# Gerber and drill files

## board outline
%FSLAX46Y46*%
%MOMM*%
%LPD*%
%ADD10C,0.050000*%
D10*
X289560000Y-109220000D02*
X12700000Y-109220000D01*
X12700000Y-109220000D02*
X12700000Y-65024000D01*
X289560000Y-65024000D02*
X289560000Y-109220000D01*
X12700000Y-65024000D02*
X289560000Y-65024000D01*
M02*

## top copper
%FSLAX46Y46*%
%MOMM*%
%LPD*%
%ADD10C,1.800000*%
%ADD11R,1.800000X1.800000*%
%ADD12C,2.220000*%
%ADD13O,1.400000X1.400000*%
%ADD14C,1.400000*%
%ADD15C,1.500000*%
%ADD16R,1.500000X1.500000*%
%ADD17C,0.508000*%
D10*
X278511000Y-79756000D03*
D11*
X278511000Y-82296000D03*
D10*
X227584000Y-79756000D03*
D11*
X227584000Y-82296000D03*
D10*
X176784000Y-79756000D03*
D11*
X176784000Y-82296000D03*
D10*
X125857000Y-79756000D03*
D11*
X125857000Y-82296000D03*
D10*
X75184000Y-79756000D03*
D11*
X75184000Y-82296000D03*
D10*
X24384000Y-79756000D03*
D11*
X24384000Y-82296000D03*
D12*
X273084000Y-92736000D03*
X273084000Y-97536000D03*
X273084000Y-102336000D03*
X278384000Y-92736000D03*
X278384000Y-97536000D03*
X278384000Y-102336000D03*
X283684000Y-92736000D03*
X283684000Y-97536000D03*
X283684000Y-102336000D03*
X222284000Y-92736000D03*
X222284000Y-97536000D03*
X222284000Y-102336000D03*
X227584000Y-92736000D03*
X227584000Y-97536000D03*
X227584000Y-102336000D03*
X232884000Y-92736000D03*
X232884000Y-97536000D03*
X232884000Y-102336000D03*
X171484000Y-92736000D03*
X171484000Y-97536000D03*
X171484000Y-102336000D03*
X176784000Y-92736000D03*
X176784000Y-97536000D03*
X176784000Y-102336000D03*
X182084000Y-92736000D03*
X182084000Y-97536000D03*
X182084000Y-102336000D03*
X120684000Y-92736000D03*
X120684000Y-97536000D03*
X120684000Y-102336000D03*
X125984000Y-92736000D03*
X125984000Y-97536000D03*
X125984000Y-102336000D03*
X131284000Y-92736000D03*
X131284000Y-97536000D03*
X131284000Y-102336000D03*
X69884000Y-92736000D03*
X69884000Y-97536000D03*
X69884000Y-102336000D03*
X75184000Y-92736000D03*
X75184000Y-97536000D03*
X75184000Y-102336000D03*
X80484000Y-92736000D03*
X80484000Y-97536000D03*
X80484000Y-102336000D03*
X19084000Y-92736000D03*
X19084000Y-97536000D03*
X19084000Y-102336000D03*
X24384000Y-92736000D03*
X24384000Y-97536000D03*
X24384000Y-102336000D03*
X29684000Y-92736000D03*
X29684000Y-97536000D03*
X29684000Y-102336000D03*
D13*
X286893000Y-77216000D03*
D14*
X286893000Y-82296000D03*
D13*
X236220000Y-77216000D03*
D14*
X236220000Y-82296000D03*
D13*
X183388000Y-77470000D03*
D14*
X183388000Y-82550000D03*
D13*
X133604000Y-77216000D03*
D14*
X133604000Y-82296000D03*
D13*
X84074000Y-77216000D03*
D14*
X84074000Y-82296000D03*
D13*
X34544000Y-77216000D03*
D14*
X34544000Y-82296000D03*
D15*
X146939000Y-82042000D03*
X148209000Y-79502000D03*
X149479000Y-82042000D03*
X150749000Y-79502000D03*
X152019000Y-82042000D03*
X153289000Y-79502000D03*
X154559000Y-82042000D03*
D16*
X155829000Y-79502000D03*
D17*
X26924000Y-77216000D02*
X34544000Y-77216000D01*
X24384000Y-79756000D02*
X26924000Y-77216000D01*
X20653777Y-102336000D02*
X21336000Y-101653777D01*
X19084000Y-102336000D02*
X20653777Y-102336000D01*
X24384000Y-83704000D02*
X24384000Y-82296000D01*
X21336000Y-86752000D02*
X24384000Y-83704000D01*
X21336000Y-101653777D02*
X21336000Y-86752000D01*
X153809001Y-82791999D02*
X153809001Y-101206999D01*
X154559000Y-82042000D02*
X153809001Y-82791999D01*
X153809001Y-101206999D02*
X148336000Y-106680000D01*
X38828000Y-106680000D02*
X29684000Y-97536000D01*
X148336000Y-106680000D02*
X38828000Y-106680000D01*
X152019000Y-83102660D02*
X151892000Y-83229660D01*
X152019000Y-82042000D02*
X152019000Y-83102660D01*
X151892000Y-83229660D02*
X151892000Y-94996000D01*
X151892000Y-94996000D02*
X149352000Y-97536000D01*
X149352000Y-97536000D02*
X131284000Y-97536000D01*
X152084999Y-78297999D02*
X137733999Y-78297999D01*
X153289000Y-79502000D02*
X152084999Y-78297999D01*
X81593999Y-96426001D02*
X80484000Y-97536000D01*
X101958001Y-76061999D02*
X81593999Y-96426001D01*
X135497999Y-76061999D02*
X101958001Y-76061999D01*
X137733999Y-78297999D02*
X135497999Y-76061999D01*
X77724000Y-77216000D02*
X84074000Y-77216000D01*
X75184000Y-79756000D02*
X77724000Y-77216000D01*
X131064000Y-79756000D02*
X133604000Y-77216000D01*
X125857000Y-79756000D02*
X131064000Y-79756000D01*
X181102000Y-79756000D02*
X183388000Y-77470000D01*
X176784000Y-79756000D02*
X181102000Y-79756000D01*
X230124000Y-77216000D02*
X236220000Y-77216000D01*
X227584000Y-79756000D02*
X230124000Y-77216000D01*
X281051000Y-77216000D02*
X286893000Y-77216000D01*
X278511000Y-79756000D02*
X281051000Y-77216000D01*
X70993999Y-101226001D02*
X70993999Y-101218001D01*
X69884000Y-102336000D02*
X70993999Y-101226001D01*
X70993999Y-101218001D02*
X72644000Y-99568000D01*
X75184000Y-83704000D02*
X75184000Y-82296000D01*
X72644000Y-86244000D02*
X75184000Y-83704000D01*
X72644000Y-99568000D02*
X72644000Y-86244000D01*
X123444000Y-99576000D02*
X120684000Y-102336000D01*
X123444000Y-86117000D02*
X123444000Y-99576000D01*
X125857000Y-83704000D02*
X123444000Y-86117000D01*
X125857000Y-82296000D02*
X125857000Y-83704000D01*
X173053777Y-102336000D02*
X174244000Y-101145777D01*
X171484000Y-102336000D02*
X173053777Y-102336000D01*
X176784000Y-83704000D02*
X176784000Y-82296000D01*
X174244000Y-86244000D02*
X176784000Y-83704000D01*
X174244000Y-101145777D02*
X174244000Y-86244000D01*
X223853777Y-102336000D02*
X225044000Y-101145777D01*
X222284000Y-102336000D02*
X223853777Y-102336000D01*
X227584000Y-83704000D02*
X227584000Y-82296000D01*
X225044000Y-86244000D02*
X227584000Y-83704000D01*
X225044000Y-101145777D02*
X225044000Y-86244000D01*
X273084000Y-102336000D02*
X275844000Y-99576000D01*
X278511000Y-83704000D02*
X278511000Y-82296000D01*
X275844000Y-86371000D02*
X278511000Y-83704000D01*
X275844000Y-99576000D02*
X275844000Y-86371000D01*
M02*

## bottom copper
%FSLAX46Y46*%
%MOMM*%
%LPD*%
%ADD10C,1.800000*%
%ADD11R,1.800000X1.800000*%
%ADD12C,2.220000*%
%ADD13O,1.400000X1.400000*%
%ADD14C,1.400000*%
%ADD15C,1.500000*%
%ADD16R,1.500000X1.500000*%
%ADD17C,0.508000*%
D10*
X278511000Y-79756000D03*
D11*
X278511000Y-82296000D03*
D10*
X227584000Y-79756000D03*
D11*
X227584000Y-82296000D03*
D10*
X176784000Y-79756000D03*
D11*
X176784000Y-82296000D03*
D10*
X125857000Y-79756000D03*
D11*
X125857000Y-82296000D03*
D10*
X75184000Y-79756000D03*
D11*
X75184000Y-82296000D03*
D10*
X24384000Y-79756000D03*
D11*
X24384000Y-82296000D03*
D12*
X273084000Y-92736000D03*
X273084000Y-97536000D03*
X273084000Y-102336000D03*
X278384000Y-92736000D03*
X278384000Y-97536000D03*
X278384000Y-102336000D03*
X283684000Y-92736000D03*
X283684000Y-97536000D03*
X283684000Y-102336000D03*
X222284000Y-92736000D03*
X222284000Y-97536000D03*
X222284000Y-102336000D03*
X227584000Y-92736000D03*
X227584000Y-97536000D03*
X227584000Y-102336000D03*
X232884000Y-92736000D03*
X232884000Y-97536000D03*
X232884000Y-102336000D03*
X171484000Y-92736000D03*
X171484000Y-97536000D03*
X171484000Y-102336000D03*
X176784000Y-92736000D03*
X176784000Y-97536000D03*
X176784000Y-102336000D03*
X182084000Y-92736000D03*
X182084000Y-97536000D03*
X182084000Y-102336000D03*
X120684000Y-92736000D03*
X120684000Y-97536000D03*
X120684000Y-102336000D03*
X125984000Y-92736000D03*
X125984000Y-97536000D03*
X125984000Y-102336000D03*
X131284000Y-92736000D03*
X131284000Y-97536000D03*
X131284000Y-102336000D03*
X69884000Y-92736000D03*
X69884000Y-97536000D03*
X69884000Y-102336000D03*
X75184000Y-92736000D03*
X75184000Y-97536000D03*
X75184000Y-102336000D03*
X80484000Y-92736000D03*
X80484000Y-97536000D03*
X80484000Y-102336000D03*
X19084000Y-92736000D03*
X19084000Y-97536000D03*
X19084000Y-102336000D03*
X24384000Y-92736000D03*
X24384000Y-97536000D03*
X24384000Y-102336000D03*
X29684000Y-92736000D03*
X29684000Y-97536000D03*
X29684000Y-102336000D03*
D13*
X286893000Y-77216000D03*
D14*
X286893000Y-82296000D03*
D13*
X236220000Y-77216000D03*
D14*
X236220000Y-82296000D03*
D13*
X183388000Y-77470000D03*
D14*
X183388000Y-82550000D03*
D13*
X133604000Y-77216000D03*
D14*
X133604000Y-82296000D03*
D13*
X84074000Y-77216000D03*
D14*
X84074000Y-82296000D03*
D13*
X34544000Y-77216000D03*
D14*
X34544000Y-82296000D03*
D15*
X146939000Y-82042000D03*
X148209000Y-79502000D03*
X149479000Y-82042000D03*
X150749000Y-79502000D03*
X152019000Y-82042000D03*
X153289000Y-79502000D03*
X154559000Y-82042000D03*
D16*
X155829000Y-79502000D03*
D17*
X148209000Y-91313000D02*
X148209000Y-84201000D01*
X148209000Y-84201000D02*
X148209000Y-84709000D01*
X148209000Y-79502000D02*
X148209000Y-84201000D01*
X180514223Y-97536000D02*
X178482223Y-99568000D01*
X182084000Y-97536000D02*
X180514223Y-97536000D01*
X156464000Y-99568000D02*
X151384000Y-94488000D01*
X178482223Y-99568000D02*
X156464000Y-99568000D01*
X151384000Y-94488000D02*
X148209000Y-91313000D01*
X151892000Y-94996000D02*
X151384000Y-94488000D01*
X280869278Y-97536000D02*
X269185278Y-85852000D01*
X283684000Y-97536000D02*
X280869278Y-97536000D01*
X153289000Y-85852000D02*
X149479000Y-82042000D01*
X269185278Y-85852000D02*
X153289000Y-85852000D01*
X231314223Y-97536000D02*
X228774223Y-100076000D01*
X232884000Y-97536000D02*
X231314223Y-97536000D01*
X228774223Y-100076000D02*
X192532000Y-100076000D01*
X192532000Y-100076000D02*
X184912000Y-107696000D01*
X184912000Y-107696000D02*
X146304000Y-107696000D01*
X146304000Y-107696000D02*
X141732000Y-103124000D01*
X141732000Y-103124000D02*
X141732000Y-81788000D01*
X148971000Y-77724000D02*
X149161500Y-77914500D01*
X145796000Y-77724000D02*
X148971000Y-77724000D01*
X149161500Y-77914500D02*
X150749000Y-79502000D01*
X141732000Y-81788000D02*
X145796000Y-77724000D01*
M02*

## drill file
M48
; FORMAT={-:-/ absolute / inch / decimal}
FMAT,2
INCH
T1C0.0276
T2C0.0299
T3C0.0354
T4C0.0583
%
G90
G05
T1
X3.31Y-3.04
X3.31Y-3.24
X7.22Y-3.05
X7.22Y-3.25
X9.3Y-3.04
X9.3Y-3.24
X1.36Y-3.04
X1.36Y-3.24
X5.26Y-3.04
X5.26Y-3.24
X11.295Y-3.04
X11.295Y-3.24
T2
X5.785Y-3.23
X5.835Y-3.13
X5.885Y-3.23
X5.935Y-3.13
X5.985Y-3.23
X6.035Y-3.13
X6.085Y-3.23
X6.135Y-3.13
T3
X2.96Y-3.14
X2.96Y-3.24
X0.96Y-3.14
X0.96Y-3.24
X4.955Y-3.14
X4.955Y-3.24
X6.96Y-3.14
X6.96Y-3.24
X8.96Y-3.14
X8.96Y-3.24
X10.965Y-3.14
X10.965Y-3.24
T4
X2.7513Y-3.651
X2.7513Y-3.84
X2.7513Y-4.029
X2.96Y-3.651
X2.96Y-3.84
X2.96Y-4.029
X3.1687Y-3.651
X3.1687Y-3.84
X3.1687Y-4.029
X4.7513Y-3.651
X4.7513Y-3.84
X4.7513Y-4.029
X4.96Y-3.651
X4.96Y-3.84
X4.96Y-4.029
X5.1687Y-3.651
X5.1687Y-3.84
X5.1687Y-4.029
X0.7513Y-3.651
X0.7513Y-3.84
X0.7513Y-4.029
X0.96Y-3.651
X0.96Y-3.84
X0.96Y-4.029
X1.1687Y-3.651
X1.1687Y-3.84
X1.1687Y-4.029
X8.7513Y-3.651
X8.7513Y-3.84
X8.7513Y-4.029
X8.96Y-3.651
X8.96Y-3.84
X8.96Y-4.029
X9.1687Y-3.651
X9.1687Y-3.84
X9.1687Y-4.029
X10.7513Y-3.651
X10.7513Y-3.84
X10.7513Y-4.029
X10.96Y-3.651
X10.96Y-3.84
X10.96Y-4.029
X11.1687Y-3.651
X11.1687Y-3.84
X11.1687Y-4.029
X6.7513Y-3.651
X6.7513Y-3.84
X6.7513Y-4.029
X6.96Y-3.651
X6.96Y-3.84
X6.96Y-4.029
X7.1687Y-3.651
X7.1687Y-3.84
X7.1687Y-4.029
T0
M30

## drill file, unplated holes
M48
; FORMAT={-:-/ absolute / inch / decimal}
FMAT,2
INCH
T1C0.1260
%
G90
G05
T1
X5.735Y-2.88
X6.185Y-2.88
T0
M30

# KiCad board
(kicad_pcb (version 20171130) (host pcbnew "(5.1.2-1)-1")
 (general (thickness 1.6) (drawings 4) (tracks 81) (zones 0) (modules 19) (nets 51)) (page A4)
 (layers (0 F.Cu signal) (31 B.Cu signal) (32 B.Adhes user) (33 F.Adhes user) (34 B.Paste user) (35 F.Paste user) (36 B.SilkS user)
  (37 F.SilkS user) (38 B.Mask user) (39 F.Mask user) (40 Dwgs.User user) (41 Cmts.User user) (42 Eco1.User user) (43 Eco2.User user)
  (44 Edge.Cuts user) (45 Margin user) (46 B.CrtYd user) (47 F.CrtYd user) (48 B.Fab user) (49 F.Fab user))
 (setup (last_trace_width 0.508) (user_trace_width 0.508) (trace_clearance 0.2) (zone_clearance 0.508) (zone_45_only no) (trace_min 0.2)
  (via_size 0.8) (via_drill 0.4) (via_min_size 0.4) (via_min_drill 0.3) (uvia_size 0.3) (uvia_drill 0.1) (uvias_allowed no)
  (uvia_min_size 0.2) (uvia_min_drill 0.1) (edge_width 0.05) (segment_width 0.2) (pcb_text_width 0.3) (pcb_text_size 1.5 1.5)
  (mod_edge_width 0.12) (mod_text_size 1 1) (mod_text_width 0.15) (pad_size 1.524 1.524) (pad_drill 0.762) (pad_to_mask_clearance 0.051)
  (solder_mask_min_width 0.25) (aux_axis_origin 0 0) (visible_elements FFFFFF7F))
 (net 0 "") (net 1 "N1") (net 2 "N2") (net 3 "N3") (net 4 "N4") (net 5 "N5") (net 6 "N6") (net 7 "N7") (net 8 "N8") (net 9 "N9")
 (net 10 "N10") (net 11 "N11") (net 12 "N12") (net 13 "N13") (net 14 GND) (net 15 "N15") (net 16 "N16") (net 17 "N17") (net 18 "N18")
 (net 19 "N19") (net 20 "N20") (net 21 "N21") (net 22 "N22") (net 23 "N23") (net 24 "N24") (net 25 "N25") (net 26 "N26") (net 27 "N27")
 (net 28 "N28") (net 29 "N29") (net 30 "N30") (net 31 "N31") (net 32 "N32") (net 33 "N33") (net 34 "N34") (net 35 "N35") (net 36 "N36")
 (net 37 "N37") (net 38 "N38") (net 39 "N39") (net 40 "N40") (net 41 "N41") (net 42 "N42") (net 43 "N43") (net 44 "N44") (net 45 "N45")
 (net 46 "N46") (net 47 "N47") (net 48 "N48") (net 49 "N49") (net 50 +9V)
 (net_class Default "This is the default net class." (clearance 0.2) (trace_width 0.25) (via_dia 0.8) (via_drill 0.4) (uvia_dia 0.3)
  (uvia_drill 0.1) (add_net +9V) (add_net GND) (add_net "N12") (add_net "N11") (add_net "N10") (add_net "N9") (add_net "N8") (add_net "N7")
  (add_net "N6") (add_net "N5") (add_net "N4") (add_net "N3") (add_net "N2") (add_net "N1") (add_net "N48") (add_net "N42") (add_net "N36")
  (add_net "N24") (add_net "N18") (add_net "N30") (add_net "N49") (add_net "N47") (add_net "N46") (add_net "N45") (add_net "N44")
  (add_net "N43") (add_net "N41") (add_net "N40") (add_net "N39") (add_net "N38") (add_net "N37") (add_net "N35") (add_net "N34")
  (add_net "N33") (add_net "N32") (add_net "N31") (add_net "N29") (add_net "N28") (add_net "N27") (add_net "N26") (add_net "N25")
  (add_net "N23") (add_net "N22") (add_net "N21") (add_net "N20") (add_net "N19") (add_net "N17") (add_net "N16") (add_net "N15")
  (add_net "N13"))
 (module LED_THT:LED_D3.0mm (layer F.Cu) (at 278.511 82.296 90)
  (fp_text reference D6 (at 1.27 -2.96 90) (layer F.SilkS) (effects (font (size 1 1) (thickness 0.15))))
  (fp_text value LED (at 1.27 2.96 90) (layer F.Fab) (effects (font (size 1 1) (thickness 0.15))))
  (pad 2 thru_hole circle (at 2.54 0 90) (size 1.8 1.8) (drill 0.9) (layers *.Cu *.Mask) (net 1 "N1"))
  (pad 1 thru_hole rect (at 0 0 90) (size 1.8 1.8) (drill 0.9) (layers *.Cu *.Mask) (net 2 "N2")))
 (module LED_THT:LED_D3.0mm (layer F.Cu) (at 227.584 82.296 90)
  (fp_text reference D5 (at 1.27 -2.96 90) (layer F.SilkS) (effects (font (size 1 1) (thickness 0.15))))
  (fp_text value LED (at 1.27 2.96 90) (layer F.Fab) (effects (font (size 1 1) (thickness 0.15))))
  (pad 2 thru_hole circle (at 2.54 0 90) (size 1.8 1.8) (drill 0.9) (layers *.Cu *.Mask) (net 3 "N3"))
  (pad 1 thru_hole rect (at 0 0 90) (size 1.8 1.8) (drill 0.9) (layers *.Cu *.Mask) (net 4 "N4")))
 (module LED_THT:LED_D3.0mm (layer F.Cu) (at 176.784 82.296 90)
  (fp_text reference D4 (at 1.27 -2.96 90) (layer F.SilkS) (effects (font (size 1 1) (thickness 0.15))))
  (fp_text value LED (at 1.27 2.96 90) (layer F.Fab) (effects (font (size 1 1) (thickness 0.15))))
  (pad 2 thru_hole circle (at 2.54 0 90) (size 1.8 1.8) (drill 0.9) (layers *.Cu *.Mask) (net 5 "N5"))
  (pad 1 thru_hole rect (at 0 0 90) (size 1.8 1.8) (drill 0.9) (layers *.Cu *.Mask) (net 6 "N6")))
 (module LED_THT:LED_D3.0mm (layer F.Cu) (at 125.857 82.296 90)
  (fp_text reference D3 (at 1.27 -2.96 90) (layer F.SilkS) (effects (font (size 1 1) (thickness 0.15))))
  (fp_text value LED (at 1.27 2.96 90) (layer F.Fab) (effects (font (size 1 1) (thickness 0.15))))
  (pad 2 thru_hole circle (at 2.54 0 90) (size 1.8 1.8) (drill 0.9) (layers *.Cu *.Mask) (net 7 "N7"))
  (pad 1 thru_hole rect (at 0 0 90) (size 1.8 1.8) (drill 0.9) (layers *.Cu *.Mask) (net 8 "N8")))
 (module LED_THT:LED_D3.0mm (layer F.Cu) (at 75.184 82.296 90)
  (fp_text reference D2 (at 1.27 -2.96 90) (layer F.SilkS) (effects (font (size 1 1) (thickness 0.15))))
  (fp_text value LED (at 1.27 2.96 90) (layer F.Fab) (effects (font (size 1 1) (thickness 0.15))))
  (pad 2 thru_hole circle (at 2.54 0 90) (size 1.8 1.8) (drill 0.9) (layers *.Cu *.Mask) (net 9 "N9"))
  (pad 1 thru_hole rect (at 0 0 90) (size 1.8 1.8) (drill 0.9) (layers *.Cu *.Mask) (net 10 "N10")))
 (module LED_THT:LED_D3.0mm (layer F.Cu) (at 24.384 82.296 90)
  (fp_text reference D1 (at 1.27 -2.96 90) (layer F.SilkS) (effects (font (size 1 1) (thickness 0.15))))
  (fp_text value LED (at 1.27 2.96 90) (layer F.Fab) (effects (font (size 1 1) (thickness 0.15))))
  (pad 2 thru_hole circle (at 2.54 0 90) (size 1.8 1.8) (drill 0.9) (layers *.Cu *.Mask) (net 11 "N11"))
  (pad 1 thru_hole rect (at 0 0 90) (size 1.8 1.8) (drill 0.9) (layers *.Cu *.Mask) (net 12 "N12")))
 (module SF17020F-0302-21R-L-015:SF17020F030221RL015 (layer F.Cu) (at 278.384 97.536)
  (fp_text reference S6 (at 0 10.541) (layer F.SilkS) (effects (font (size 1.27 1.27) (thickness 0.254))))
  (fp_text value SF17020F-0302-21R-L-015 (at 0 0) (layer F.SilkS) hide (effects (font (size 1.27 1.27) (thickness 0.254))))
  (pad 9 thru_hole circle (at -5.3 -4.8 90) (size 2.22 2.22) (drill 1.48) (layers *.Cu *.Mask F.SilkS) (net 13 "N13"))
  (pad 8 thru_hole circle (at -5.3 0 90) (size 2.22 2.22) (drill 1.48) (layers *.Cu *.Mask F.SilkS) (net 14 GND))
  (pad 7 thru_hole circle (at -5.3 4.8 90) (size 2.22 2.22) (drill 1.48) (layers *.Cu *.Mask F.SilkS) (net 2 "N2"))
  (pad 6 thru_hole circle (at 0 -4.8 90) (size 2.22 2.22) (drill 1.48) (layers *.Cu *.Mask F.SilkS) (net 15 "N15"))
  (pad 5 thru_hole circle (at 0 0 90) (size 2.22 2.22) (drill 1.48) (layers *.Cu *.Mask F.SilkS) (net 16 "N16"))
  (pad 4 thru_hole circle (at 0 4.8 90) (size 2.22 2.22) (drill 1.48) (layers *.Cu *.Mask F.SilkS) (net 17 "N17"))
  (pad 3 thru_hole circle (at 5.3 -4.8 90) (size 2.22 2.22) (drill 1.48) (layers *.Cu *.Mask F.SilkS) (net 14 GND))
  (pad 2 thru_hole circle (at 5.3 0 90) (size 2.22 2.22) (drill 1.48) (layers *.Cu *.Mask F.SilkS) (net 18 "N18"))
  (pad 1 thru_hole circle (at 5.3 4.8 90) (size 2.22 2.22) (drill 1.48) (layers *.Cu *.Mask F.SilkS) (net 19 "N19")))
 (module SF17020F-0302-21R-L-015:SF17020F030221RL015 (layer F.Cu) (at 227.584 97.536)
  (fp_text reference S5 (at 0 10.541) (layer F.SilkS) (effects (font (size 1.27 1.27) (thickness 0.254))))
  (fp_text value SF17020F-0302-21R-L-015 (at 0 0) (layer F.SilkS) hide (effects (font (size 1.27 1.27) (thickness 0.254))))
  (pad 9 thru_hole circle (at -5.3 -4.8 90) (size 2.22 2.22) (drill 1.48) (layers *.Cu *.Mask F.SilkS) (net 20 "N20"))
  (pad 8 thru_hole circle (at -5.3 0 90) (size 2.22 2.22) (drill 1.48) (layers *.Cu *.Mask F.SilkS) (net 14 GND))
  (pad 7 thru_hole circle (at -5.3 4.8 90) (size 2.22 2.22) (drill 1.48) (layers *.Cu *.Mask F.SilkS) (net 4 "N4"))
  (pad 6 thru_hole circle (at 0 -4.8 90) (size 2.22 2.22) (drill 1.48) (layers *.Cu *.Mask F.SilkS) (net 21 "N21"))
  (pad 5 thru_hole circle (at 0 0 90) (size 2.22 2.22) (drill 1.48) (layers *.Cu *.Mask F.SilkS) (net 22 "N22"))
  (pad 4 thru_hole circle (at 0 4.8 90) (size 2.22 2.22) (drill 1.48) (layers *.Cu *.Mask F.SilkS) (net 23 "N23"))
  (pad 3 thru_hole circle (at 5.3 -4.8 90) (size 2.22 2.22) (drill 1.48) (layers *.Cu *.Mask F.SilkS) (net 14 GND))
  (pad 2 thru_hole circle (at 5.3 0 90) (size 2.22 2.22) (drill 1.48) (layers *.Cu *.Mask F.SilkS) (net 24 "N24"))
  (pad 1 thru_hole circle (at 5.3 4.8 90) (size 2.22 2.22) (drill 1.48) (layers *.Cu *.Mask F.SilkS) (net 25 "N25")))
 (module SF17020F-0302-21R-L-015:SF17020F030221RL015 (layer F.Cu) (at 176.784 97.536)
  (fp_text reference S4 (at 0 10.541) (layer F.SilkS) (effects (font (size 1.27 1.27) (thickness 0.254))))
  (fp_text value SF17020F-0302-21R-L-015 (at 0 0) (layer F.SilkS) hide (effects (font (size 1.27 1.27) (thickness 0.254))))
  (pad 9 thru_hole circle (at -5.3 -4.8 90) (size 2.22 2.22) (drill 1.48) (layers *.Cu *.Mask F.SilkS) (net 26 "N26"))
  (pad 8 thru_hole circle (at -5.3 0 90) (size 2.22 2.22) (drill 1.48) (layers *.Cu *.Mask F.SilkS) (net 14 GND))
  (pad 7 thru_hole circle (at -5.3 4.8 90) (size 2.22 2.22) (drill 1.48) (layers *.Cu *.Mask F.SilkS) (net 6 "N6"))
  (pad 6 thru_hole circle (at 0 -4.8 90) (size 2.22 2.22) (drill 1.48) (layers *.Cu *.Mask F.SilkS) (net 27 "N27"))
  (pad 5 thru_hole circle (at 0 0 90) (size 2.22 2.22) (drill 1.48) (layers *.Cu *.Mask F.SilkS) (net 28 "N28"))
  (pad 4 thru_hole circle (at 0 4.8 90) (size 2.22 2.22) (drill 1.48) (layers *.Cu *.Mask F.SilkS) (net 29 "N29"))
  (pad 3 thru_hole circle (at 5.3 -4.8 90) (size 2.22 2.22) (drill 1.48) (layers *.Cu *.Mask F.SilkS) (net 14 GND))
  (pad 2 thru_hole circle (at 5.3 0 90) (size 2.22 2.22) (drill 1.48) (layers *.Cu *.Mask F.SilkS) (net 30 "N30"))
  (pad 1 thru_hole circle (at 5.3 4.8 90) (size 2.22 2.22) (drill 1.48) (layers *.Cu *.Mask F.SilkS) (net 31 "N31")))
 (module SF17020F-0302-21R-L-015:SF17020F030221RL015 (layer F.Cu) (at 125.984 97.536)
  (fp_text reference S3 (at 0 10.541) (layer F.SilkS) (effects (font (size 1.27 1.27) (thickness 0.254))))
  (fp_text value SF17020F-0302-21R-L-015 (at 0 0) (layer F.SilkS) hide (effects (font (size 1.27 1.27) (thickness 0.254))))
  (pad 9 thru_hole circle (at -5.3 -4.8 90) (size 2.22 2.22) (drill 1.48) (layers *.Cu *.Mask F.SilkS) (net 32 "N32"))
  (pad 8 thru_hole circle (at -5.3 0 90) (size 2.22 2.22) (drill 1.48) (layers *.Cu *.Mask F.SilkS) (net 14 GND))
  (pad 7 thru_hole circle (at -5.3 4.8 90) (size 2.22 2.22) (drill 1.48) (layers *.Cu *.Mask F.SilkS) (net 8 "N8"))
  (pad 6 thru_hole circle (at 0 -4.8 90) (size 2.22 2.22) (drill 1.48) (layers *.Cu *.Mask F.SilkS) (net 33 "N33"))
  (pad 5 thru_hole circle (at 0 0 90) (size 2.22 2.22) (drill 1.48) (layers *.Cu *.Mask F.SilkS) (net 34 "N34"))
  (pad 4 thru_hole circle (at 0 4.8 90) (size 2.22 2.22) (drill 1.48) (layers *.Cu *.Mask F.SilkS) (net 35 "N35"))
  (pad 3 thru_hole circle (at 5.3 -4.8 90) (size 2.22 2.22) (drill 1.48) (layers *.Cu *.Mask F.SilkS) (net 14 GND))
  (pad 2 thru_hole circle (at 5.3 0 90) (size 2.22 2.22) (drill 1.48) (layers *.Cu *.Mask F.SilkS) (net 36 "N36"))
  (pad 1 thru_hole circle (at 5.3 4.8 90) (size 2.22 2.22) (drill 1.48) (layers *.Cu *.Mask F.SilkS) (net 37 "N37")))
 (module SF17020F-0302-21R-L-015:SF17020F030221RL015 (layer F.Cu) (at 75.184 97.536)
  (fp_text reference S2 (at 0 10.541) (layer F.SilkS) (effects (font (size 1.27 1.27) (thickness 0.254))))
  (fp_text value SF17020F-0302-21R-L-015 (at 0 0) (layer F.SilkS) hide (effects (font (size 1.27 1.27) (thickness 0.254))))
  (pad 9 thru_hole circle (at -5.3 -4.8 90) (size 2.22 2.22) (drill 1.48) (layers *.Cu *.Mask F.SilkS) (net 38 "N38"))
  (pad 8 thru_hole circle (at -5.3 0 90) (size 2.22 2.22) (drill 1.48) (layers *.Cu *.Mask F.SilkS) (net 14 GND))
  (pad 7 thru_hole circle (at -5.3 4.8 90) (size 2.22 2.22) (drill 1.48) (layers *.Cu *.Mask F.SilkS) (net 10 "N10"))
  (pad 6 thru_hole circle (at 0 -4.8 90) (size 2.22 2.22) (drill 1.48) (layers *.Cu *.Mask F.SilkS) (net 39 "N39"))
  (pad 5 thru_hole circle (at 0 0 90) (size 2.22 2.22) (drill 1.48) (layers *.Cu *.Mask F.SilkS) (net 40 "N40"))
  (pad 4 thru_hole circle (at 0 4.8 90) (size 2.22 2.22) (drill 1.48) (layers *.Cu *.Mask F.SilkS) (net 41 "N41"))
  (pad 3 thru_hole circle (at 5.3 -4.8 90) (size 2.22 2.22) (drill 1.48) (layers *.Cu *.Mask F.SilkS) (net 14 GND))
  (pad 2 thru_hole circle (at 5.3 0 90) (size 2.22 2.22) (drill 1.48) (layers *.Cu *.Mask F.SilkS) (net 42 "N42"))
  (pad 1 thru_hole circle (at 5.3 4.8 90) (size 2.22 2.22) (drill 1.48) (layers *.Cu *.Mask F.SilkS) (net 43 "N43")))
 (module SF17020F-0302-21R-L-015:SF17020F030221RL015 (layer F.Cu) (at 24.384 97.536)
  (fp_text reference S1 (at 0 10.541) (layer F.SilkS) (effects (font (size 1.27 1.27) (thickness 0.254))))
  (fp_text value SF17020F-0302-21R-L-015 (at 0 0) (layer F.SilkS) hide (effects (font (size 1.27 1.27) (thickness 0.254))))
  (pad 9 thru_hole circle (at -5.3 -4.8 90) (size 2.22 2.22) (drill 1.48) (layers *.Cu *.Mask F.SilkS) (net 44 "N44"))
  (pad 8 thru_hole circle (at -5.3 0 90) (size 2.22 2.22) (drill 1.48) (layers *.Cu *.Mask F.SilkS) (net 14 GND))
  (pad 7 thru_hole circle (at -5.3 4.8 90) (size 2.22 2.22) (drill 1.48) (layers *.Cu *.Mask F.SilkS) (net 12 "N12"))
  (pad 6 thru_hole circle (at 0 -4.8 90) (size 2.22 2.22) (drill 1.48) (layers *.Cu *.Mask F.SilkS) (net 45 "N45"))
  (pad 5 thru_hole circle (at 0 0 90) (size 2.22 2.22) (drill 1.48) (layers *.Cu *.Mask F.SilkS) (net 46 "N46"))
  (pad 4 thru_hole circle (at 0 4.8 90) (size 2.22 2.22) (drill 1.48) (layers *.Cu *.Mask F.SilkS) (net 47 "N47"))
  (pad 3 thru_hole circle (at 5.3 -4.8 90) (size 2.22 2.22) (drill 1.48) (layers *.Cu *.Mask F.SilkS) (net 14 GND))
  (pad 2 thru_hole circle (at 5.3 0 90) (size 2.22 2.22) (drill 1.48) (layers *.Cu *.Mask F.SilkS) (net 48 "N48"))
  (pad 1 thru_hole circle (at 5.3 4.8 90) (size 2.22 2.22) (drill 1.48) (layers *.Cu *.Mask F.SilkS) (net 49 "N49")))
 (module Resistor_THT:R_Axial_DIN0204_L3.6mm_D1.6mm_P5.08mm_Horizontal (layer F.Cu) (at 286.893 82.296 90)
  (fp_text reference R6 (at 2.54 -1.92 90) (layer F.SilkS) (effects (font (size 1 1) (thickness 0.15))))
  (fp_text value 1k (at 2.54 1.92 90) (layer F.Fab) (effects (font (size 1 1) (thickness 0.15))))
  (pad 2 thru_hole oval (at 5.08 0 90) (size 1.4 1.4) (drill 0.7) (layers *.Cu *.Mask) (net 1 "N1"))
  (pad 1 thru_hole circle (at 0 0 90) (size 1.4 1.4) (drill 0.7) (layers *.Cu *.Mask) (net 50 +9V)))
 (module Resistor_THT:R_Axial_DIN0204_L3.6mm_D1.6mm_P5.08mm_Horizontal (layer F.Cu) (at 236.22 82.296 90)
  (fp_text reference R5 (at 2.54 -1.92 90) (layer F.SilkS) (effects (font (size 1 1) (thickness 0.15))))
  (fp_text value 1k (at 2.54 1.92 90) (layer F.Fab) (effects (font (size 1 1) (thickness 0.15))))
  (pad 2 thru_hole oval (at 5.08 0 90) (size 1.4 1.4) (drill 0.7) (layers *.Cu *.Mask) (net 3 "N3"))
  (pad 1 thru_hole circle (at 0 0 90) (size 1.4 1.4) (drill 0.7) (layers *.Cu *.Mask) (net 50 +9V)))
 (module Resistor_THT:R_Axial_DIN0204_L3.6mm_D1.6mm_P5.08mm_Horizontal (layer F.Cu) (at 183.388 82.55 90)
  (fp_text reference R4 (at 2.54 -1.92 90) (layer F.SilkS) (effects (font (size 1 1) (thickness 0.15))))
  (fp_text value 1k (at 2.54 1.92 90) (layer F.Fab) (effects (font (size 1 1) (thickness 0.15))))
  (pad 2 thru_hole oval (at 5.08 0 90) (size 1.4 1.4) (drill 0.7) (layers *.Cu *.Mask) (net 5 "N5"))
  (pad 1 thru_hole circle (at 0 0 90) (size 1.4 1.4) (drill 0.7) (layers *.Cu *.Mask) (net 50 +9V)))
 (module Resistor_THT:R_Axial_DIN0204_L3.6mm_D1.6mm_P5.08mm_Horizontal (layer F.Cu) (at 133.604 82.296 90)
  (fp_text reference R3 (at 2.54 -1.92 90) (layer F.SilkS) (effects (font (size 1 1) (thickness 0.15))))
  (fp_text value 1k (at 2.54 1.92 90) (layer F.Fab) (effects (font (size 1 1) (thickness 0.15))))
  (pad 2 thru_hole oval (at 5.08 0 90) (size 1.4 1.4) (drill 0.7) (layers *.Cu *.Mask) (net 7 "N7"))
  (pad 1 thru_hole circle (at 0 0 90) (size 1.4 1.4) (drill 0.7) (layers *.Cu *.Mask) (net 50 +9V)))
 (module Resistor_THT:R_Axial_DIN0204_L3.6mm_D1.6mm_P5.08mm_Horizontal (layer F.Cu) (at 84.074 82.296 90)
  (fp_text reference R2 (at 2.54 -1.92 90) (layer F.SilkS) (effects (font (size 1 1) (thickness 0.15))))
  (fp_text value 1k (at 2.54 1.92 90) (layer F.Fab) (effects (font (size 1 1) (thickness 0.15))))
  (pad 2 thru_hole oval (at 5.08 0 90) (size 1.4 1.4) (drill 0.7) (layers *.Cu *.Mask) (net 9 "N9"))
  (pad 1 thru_hole circle (at 0 0 90) (size 1.4 1.4) (drill 0.7) (layers *.Cu *.Mask) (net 50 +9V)))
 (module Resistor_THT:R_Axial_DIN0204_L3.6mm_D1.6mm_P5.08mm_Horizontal (layer F.Cu) (at 34.544 82.296 90)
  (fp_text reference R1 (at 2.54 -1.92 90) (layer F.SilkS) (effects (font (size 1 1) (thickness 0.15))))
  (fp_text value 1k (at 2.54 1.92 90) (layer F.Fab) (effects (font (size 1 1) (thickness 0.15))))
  (pad 2 thru_hole oval (at 5.08 0 90) (size 1.4 1.4) (drill 0.7) (layers *.Cu *.Mask) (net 11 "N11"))
  (pad 1 thru_hole circle (at 0 0 90) (size 1.4 1.4) (drill 0.7) (layers *.Cu *.Mask) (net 50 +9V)))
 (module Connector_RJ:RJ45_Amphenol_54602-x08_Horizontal (layer F.Cu) (at 155.829 79.502 180)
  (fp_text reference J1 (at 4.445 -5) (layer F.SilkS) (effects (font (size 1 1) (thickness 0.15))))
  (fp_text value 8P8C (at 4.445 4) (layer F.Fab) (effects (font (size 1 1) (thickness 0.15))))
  (pad 8 thru_hole circle (at 8.89 -2.54 180) (size 1.5 1.5) (drill 0.76) (layers *.Cu *.Mask) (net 14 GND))
  (pad 7 thru_hole circle (at 7.62 0 180) (size 1.5 1.5) (drill 0.76) (layers *.Cu *.Mask) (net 30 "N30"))
  (pad 6 thru_hole circle (at 6.35 -2.54 180) (size 1.5 1.5) (drill 0.76) (layers *.Cu *.Mask) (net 18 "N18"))
  (pad 5 thru_hole circle (at 5.08 0 180) (size 1.5 1.5) (drill 0.76) (layers *.Cu *.Mask) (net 24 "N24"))
  (pad 4 thru_hole circle (at 3.81 -2.54 180) (size 1.5 1.5) (drill 0.76) (layers *.Cu *.Mask) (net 36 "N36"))
  (pad 3 thru_hole circle (at 2.54 0 180) (size 1.5 1.5) (drill 0.76) (layers *.Cu *.Mask) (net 42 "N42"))
  (pad 2 thru_hole circle (at 1.27 -2.54 180) (size 1.5 1.5) (drill 0.76) (layers *.Cu *.Mask) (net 48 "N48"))
  (pad 1 thru_hole rect (at 0 0 180) (size 1.5 1.5) (drill 0.76) (layers *.Cu *.Mask) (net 50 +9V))
  (pad "" np_thru_hole circle (at -1.27 6.35 180) (size 3.2 3.2) (drill 3.2) (layers *.Cu *.Mask))
  (pad "" np_thru_hole circle (at 10.16 6.35 180) (size 3.2 3.2) (drill 3.2) (layers *.Cu *.Mask)))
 (gr_line (start 289.56 109.22) (end 12.7 109.22) (layer Edge.Cuts) (width 0.05))
 (gr_line (start 12.7 109.22) (end 12.7 65.024) (layer Edge.Cuts) (width 0.05))
 (gr_line (start 289.56 65.024) (end 289.56 109.22) (layer Edge.Cuts) (width 0.05))
 (gr_line (start 12.7 65.024) (end 289.56 65.024) (layer Edge.Cuts) (width 0.05))
 (segment (start 26.924 77.216) (end 34.544 77.216) (width 0.508) (layer F.Cu) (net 11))
 (segment (start 24.384 79.756) (end 26.924 77.216) (width 0.508) (layer F.Cu) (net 11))
 (segment (start 20.653777 102.336) (end 21.336 101.653777) (width 0.508) (layer F.Cu) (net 12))
 (segment (start 19.084 102.336) (end 20.653777 102.336) (width 0.508) (layer F.Cu) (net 12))
 (segment (start 24.384 83.704) (end 24.384 82.296) (width 0.508) (layer F.Cu) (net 12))
 (segment (start 21.336 86.752) (end 24.384 83.704) (width 0.508) (layer F.Cu) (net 12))
 (segment (start 21.336 101.653777) (end 21.336 86.752) (width 0.508) (layer F.Cu) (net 12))
 (segment (start 153.809001 82.791999) (end 153.809001 101.206999) (width 0.508) (layer F.Cu) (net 48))
 (segment (start 154.559 82.042) (end 153.809001 82.791999) (width 0.508) (layer F.Cu) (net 48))
 (segment (start 153.809001 101.206999) (end 148.336 106.68) (width 0.508) (layer F.Cu) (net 48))
 (segment (start 38.828 106.68) (end 29.684 97.536) (width 0.508) (layer F.Cu) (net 48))
 (segment (start 148.336 106.68) (end 38.828 106.68) (width 0.508) (layer F.Cu) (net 48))
 (segment (start 148.209 91.313) (end 148.209 84.201) (width 0.508) (layer B.Cu) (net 30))
 (segment (start 148.209 84.201) (end 148.209 84.709) (width 0.508) (layer B.Cu) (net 30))
 (segment (start 148.209 79.502) (end 148.209 84.201) (width 0.508) (layer B.Cu) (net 30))
 (segment (start 180.514223 97.536) (end 178.482223 99.568) (width 0.508) (layer B.Cu) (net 30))
 (segment (start 182.084 97.536) (end 180.514223 97.536) (width 0.508) (layer B.Cu) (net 30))
 (segment (start 156.464 99.568) (end 151.384 94.488) (width 0.508) (layer B.Cu) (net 30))
 (segment (start 178.482223 99.568) (end 156.464 99.568) (width 0.508) (layer B.Cu) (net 30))
 (segment (start 151.384 94.488) (end 148.209 91.313) (width 0.508) (layer B.Cu) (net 30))
 (segment (start 151.892 94.996) (end 151.384 94.488) (width 0.508) (layer B.Cu) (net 30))
 (segment (start 280.869278 97.536) (end 269.185278 85.852) (width 0.508) (layer B.Cu) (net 18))
 (segment (start 283.684 97.536) (end 280.869278 97.536) (width 0.508) (layer B.Cu) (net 18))
 (segment (start 153.289 85.852) (end 149.479 82.042) (width 0.508) (layer B.Cu) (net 18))
 (segment (start 269.185278 85.852) (end 153.289 85.852) (width 0.508) (layer B.Cu) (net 18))
 (segment (start 231.314223 97.536) (end 228.774223 100.076) (width 0.508) (layer B.Cu) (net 24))
 (segment (start 232.884 97.536) (end 231.314223 97.536) (width 0.508) (layer B.Cu) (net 24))
 (segment (start 228.774223 100.076) (end 192.532 100.076) (width 0.508) (layer B.Cu) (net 24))
 (segment (start 192.532 100.076) (end 184.912 107.696) (width 0.508) (layer B.Cu) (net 24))
 (segment (start 184.912 107.696) (end 146.304 107.696) (width 0.508) (layer B.Cu) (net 24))
 (segment (start 146.304 107.696) (end 141.732 103.124) (width 0.508) (layer B.Cu) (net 24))
 (segment (start 141.732 103.124) (end 141.732 81.788) (width 0.508) (layer B.Cu) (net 24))
 (segment (start 148.971 77.724) (end 149.1615 77.9145) (width 0.508) (layer B.Cu) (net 24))
 (segment (start 145.796 77.724) (end 148.971 77.724) (width 0.508) (layer B.Cu) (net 24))
 (segment (start 149.1615 77.9145) (end 150.749 79.502) (width 0.508) (layer B.Cu) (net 24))
 (segment (start 141.732 81.788) (end 145.796 77.724) (width 0.508) (layer B.Cu) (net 24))
 (segment (start 152.019 83.10266) (end 151.892 83.22966) (width 0.508) (layer F.Cu) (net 36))
 (segment (start 152.019 82.042) (end 152.019 83.10266) (width 0.508) (layer F.Cu) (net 36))
 (segment (start 151.892 83.22966) (end 151.892 94.996) (width 0.508) (layer F.Cu) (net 36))
 (segment (start 151.892 94.996) (end 149.352 97.536) (width 0.508) (layer F.Cu) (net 36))
 (segment (start 149.352 97.536) (end 131.284 97.536) (width 0.508) (layer F.Cu) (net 36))
 (segment (start 152.084999 78.297999) (end 137.733999 78.297999) (width 0.508) (layer F.Cu) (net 42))
 (segment (start 153.289 79.502) (end 152.084999 78.297999) (width 0.508) (layer F.Cu) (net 42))
 (segment (start 81.593999 96.426001) (end 80.484 97.536) (width 0.508) (layer F.Cu) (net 42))
 (segment (start 101.958001 76.061999) (end 81.593999 96.426001) (width 0.508) (layer F.Cu) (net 42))
 (segment (start 135.497999 76.061999) (end 101.958001 76.061999) (width 0.508) (layer F.Cu) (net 42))
 (segment (start 137.733999 78.297999) (end 135.497999 76.061999) (width 0.508) (layer F.Cu) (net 42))
 (segment (start 77.724 77.216) (end 84.074 77.216) (width 0.508) (layer F.Cu) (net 9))
 (segment (start 75.184 79.756) (end 77.724 77.216) (width 0.508) (layer F.Cu) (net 9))
 (segment (start 131.064 79.756) (end 133.604 77.216) (width 0.508) (layer F.Cu) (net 7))
 (segment (start 125.857 79.756) (end 131.064 79.756) (width 0.508) (layer F.Cu) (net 7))
 (segment (start 181.102 79.756) (end 183.388 77.47) (width 0.508) (layer F.Cu) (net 5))
 (segment (start 176.784 79.756) (end 181.102 79.756) (width 0.508) (layer F.Cu) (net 5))
 (segment (start 230.124 77.216) (end 236.22 77.216) (width 0.508) (layer F.Cu) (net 3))
 (segment (start 227.584 79.756) (end 230.124 77.216) (width 0.508) (layer F.Cu) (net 3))
 (segment (start 281.051 77.216) (end 286.893 77.216) (width 0.508) (layer F.Cu) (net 1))
 (segment (start 278.511 79.756) (end 281.051 77.216) (width 0.508) (layer F.Cu) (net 1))
 (segment (start 70.993999 101.226001) (end 70.993999 101.218001) (width 0.508) (layer F.Cu) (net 10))
 (segment (start 69.884 102.336) (end 70.993999 101.226001) (width 0.508) (layer F.Cu) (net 10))
 (segment (start 70.993999 101.218001) (end 72.644 99.568) (width 0.508) (layer F.Cu) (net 10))
 (segment (start 75.184 83.704) (end 75.184 82.296) (width 0.508) (layer F.Cu) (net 10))
 (segment (start 72.644 86.244) (end 75.184 83.704) (width 0.508) (layer F.Cu) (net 10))
 (segment (start 72.644 99.568) (end 72.644 86.244) (width 0.508) (layer F.Cu) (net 10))
 (segment (start 123.444 99.576) (end 120.684 102.336) (width 0.508) (layer F.Cu) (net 8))
 (segment (start 123.444 86.117) (end 123.444 99.576) (width 0.508) (layer F.Cu) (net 8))
 (segment (start 125.857 83.704) (end 123.444 86.117) (width 0.508) (layer F.Cu) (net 8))
 (segment (start 125.857 82.296) (end 125.857 83.704) (width 0.508) (layer F.Cu) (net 8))
 (segment (start 173.053777 102.336) (end 174.244 101.145777) (width 0.508) (layer F.Cu) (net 6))
 (segment (start 171.484 102.336) (end 173.053777 102.336) (width 0.508) (layer F.Cu) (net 6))
 (segment (start 176.784 83.704) (end 176.784 82.296) (width 0.508) (layer F.Cu) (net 6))
 (segment (start 174.244 86.244) (end 176.784 83.704) (width 0.508) (layer F.Cu) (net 6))
 (segment (start 174.244 101.145777) (end 174.244 86.244) (width 0.508) (layer F.Cu) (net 6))
 (segment (start 223.853777 102.336) (end 225.044 101.145777) (width 0.508) (layer F.Cu) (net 4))
 (segment (start 222.284 102.336) (end 223.853777 102.336) (width 0.508) (layer F.Cu) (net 4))
 (segment (start 227.584 83.704) (end 227.584 82.296) (width 0.508) (layer F.Cu) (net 4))
 (segment (start 225.044 86.244) (end 227.584 83.704) (width 0.508) (layer F.Cu) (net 4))
 (segment (start 225.044 101.145777) (end 225.044 86.244) (width 0.508) (layer F.Cu) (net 4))
 (segment (start 273.084 102.336) (end 275.844 99.576) (width 0.508) (layer F.Cu) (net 2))
 (segment (start 278.511 83.704) (end 278.511 82.296) (width 0.508) (layer F.Cu) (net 2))
 (segment (start 275.844 86.371) (end 278.511 83.704) (width 0.508) (layer F.Cu) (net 2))
 (segment (start 275.844 99.576) (end 275.844 86.371) (width 0.508) (layer F.Cu) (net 2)))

